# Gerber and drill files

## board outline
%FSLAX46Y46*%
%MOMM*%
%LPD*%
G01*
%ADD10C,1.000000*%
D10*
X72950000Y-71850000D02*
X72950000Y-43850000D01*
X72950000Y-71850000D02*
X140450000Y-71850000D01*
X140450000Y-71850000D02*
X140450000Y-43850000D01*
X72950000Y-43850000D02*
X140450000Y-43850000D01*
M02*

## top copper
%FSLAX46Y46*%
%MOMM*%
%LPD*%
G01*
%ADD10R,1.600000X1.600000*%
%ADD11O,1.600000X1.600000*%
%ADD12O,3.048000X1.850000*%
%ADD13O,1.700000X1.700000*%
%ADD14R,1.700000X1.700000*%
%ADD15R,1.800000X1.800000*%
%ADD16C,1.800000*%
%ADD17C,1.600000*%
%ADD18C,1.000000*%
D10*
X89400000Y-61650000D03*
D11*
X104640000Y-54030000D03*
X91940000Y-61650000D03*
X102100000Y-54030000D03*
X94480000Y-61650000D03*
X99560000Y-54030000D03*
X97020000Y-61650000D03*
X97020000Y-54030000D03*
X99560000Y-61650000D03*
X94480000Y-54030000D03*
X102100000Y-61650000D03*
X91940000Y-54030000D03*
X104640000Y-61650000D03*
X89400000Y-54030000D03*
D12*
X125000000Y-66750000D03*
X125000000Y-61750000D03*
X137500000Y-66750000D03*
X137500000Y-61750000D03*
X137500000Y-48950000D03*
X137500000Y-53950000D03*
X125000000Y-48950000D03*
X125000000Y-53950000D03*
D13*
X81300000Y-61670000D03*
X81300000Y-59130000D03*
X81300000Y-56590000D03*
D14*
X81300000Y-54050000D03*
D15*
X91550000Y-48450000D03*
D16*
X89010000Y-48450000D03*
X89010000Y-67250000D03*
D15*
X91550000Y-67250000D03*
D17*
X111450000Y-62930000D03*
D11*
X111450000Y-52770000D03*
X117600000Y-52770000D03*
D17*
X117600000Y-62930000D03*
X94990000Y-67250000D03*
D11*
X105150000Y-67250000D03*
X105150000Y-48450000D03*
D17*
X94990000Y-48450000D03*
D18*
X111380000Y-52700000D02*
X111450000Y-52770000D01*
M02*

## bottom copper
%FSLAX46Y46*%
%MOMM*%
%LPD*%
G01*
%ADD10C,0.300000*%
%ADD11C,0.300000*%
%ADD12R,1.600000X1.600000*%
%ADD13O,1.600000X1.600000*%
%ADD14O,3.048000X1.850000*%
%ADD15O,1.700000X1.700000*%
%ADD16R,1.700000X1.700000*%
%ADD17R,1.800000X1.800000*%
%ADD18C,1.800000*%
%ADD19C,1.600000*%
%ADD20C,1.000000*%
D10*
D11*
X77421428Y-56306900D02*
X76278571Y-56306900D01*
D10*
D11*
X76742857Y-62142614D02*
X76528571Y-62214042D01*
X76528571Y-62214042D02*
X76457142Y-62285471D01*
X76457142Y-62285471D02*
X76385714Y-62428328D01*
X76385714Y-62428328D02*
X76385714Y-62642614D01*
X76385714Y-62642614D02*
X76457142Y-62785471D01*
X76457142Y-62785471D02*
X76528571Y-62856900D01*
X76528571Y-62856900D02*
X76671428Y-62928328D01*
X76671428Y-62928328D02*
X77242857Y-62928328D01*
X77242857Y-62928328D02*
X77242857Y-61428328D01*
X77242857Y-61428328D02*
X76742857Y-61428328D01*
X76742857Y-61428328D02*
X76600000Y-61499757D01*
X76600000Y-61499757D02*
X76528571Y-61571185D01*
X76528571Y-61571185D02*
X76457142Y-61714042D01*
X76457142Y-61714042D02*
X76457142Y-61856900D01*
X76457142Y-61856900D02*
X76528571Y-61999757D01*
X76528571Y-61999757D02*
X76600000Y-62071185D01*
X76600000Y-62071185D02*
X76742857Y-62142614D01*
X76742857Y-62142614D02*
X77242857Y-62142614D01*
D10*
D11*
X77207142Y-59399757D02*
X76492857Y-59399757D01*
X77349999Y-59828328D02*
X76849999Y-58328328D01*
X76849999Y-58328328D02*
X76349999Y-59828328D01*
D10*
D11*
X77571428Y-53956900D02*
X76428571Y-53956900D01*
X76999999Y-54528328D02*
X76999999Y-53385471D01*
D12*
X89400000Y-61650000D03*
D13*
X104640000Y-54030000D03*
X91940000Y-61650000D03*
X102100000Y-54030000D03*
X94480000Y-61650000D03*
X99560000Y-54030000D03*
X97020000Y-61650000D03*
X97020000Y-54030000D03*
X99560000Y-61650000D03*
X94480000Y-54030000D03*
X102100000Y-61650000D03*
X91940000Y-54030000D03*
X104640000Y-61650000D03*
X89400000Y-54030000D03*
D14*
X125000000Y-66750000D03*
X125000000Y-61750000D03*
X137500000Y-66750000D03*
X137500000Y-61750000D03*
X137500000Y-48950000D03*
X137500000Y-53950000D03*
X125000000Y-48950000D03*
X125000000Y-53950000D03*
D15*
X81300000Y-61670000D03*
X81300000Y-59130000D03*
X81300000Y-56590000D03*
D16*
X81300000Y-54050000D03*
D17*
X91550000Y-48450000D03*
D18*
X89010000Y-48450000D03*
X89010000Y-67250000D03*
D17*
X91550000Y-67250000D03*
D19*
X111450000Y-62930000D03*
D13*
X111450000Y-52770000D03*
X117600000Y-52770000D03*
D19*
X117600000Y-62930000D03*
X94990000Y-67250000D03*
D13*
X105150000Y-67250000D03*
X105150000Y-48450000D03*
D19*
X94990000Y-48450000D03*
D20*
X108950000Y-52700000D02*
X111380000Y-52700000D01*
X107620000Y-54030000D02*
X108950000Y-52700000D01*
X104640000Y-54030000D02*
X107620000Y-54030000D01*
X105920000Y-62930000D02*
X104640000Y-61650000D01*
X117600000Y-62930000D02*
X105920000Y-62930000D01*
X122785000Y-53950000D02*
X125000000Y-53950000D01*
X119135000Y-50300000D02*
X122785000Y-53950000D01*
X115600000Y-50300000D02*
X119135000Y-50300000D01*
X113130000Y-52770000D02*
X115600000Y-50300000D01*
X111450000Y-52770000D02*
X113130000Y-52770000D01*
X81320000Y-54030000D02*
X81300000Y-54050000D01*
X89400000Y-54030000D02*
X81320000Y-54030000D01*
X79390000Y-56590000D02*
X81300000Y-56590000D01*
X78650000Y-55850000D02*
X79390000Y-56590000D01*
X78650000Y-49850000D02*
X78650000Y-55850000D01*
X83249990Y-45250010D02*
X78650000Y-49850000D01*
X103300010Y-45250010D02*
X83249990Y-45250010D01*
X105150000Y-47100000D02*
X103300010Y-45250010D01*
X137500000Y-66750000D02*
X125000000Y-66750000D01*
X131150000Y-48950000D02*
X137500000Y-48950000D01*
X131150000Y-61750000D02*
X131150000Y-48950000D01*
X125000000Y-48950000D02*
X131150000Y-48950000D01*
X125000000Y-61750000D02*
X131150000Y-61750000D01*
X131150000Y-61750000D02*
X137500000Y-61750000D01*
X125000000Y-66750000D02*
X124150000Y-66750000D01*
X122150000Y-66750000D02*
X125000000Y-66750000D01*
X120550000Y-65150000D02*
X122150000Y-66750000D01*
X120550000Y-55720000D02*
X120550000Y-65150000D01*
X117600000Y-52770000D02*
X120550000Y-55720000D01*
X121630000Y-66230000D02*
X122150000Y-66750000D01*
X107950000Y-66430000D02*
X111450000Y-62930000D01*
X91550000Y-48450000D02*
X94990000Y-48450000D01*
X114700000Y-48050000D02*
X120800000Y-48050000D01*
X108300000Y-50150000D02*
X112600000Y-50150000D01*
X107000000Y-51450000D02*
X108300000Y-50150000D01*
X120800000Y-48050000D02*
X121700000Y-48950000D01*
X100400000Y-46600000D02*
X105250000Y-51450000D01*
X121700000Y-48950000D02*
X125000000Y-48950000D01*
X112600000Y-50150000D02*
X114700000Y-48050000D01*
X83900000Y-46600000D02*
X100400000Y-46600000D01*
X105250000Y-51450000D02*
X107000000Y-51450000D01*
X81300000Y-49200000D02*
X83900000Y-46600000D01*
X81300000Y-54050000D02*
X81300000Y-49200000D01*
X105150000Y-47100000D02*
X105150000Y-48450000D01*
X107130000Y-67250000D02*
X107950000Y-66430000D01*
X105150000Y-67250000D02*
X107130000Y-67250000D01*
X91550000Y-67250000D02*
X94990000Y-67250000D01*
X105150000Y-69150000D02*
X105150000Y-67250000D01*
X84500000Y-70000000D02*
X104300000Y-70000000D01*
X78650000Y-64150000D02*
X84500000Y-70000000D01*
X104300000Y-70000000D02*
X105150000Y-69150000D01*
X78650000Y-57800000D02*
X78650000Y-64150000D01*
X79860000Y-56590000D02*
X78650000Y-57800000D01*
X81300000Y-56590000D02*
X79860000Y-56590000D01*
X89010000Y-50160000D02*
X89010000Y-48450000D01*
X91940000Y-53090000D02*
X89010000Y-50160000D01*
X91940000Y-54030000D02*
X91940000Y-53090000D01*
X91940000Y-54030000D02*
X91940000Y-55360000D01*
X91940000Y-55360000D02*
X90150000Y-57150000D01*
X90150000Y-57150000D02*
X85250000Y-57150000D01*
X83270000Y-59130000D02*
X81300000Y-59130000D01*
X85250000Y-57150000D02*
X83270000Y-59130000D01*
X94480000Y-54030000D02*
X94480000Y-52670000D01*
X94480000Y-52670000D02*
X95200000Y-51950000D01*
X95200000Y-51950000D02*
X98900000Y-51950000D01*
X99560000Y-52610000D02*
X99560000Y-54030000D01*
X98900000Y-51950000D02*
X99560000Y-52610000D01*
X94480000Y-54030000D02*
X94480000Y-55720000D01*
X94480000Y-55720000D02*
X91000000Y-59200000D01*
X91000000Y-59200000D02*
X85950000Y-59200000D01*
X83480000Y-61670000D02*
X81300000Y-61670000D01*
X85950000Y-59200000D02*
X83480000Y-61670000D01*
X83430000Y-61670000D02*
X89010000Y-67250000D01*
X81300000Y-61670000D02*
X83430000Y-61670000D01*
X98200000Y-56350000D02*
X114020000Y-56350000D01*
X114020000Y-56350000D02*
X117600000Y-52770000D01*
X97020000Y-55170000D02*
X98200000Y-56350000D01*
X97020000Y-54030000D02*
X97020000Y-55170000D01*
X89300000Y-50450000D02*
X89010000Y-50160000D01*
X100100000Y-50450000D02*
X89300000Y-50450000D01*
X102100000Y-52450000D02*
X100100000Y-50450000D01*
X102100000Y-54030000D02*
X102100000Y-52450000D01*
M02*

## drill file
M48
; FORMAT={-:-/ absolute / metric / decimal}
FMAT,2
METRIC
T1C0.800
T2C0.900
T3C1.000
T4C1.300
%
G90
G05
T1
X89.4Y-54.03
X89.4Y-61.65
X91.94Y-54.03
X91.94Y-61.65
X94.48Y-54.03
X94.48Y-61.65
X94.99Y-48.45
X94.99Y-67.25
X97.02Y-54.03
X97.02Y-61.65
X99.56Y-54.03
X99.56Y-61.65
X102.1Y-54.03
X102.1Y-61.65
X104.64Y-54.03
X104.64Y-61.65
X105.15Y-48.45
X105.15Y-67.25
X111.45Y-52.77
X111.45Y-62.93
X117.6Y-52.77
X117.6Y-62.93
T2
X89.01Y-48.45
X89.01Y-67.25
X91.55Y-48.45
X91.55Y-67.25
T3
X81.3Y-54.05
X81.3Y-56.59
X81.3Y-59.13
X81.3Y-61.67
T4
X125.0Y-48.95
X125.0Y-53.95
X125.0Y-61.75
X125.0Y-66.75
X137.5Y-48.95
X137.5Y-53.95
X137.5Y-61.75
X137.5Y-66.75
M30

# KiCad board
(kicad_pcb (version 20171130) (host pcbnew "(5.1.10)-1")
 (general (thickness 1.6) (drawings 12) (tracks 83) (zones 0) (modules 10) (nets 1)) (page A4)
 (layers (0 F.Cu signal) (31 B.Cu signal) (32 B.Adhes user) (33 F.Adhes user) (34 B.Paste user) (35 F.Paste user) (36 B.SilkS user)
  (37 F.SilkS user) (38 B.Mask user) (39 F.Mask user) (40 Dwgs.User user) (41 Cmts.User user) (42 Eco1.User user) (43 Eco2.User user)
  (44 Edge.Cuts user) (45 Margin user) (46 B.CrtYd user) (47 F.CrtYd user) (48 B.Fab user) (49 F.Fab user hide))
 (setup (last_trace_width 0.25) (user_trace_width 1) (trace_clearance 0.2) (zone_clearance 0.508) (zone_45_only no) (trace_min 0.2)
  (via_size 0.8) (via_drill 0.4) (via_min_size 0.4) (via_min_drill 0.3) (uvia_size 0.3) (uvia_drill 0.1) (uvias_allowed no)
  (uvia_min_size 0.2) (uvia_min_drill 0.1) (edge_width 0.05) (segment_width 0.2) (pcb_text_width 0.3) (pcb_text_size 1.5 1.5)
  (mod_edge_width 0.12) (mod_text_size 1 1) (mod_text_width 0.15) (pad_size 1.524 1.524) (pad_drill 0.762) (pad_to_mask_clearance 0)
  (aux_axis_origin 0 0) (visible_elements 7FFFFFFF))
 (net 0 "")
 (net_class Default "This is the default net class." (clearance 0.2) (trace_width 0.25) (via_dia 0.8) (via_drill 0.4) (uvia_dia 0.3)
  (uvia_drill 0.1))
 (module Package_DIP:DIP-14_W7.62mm (layer F.Cu) (at 89.4 61.65 90)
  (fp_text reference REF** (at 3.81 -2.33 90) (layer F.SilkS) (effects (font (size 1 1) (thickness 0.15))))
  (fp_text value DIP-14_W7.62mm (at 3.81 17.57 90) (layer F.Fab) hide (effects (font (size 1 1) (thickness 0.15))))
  (pad 1 thru_hole rect (at 0 0 90) (size 1.6 1.6) (drill 0.8) (layers *.Cu *.Mask))
  (pad 8 thru_hole oval (at 7.62 15.24 90) (size 1.6 1.6) (drill 0.8) (layers *.Cu *.Mask))
  (pad 2 thru_hole oval (at 0 2.54 90) (size 1.6 1.6) (drill 0.8) (layers *.Cu *.Mask))
  (pad 9 thru_hole oval (at 7.62 12.7 90) (size 1.6 1.6) (drill 0.8) (layers *.Cu *.Mask))
  (pad 3 thru_hole oval (at 0 5.08 90) (size 1.6 1.6) (drill 0.8) (layers *.Cu *.Mask))
  (pad 10 thru_hole oval (at 7.62 10.16 90) (size 1.6 1.6) (drill 0.8) (layers *.Cu *.Mask))
  (pad 4 thru_hole oval (at 0 7.62 90) (size 1.6 1.6) (drill 0.8) (layers *.Cu *.Mask))
  (pad 11 thru_hole oval (at 7.62 7.62 90) (size 1.6 1.6) (drill 0.8) (layers *.Cu *.Mask))
  (pad 5 thru_hole oval (at 0 10.16 90) (size 1.6 1.6) (drill 0.8) (layers *.Cu *.Mask))
  (pad 12 thru_hole oval (at 7.62 5.08 90) (size 1.6 1.6) (drill 0.8) (layers *.Cu *.Mask))
  (pad 6 thru_hole oval (at 0 12.7 90) (size 1.6 1.6) (drill 0.8) (layers *.Cu *.Mask))
  (pad 13 thru_hole oval (at 7.62 2.54 90) (size 1.6 1.6) (drill 0.8) (layers *.Cu *.Mask))
  (pad 7 thru_hole oval (at 0 15.24 90) (size 1.6 1.6) (drill 0.8) (layers *.Cu *.Mask))
  (pad 14 thru_hole oval (at 7.62 0 90) (size 1.6 1.6) (drill 0.8) (layers *.Cu *.Mask)))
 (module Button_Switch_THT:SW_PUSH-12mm (layer F.Cu) (at 137.5 66.75 180)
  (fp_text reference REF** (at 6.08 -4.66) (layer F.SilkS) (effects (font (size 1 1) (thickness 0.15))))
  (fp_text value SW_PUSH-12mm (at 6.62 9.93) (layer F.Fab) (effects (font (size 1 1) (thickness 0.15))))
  (pad 1 thru_hole oval (at 12.5 0 180) (size 3.048 1.85) (drill 1.3) (layers *.Cu *.Mask))
  (pad 2 thru_hole oval (at 12.5 5 180) (size 3.048 1.85) (drill 1.3) (layers *.Cu *.Mask))
  (pad 1 thru_hole oval (at 0 0 180) (size 3.048 1.85) (drill 1.3) (layers *.Cu *.Mask))
  (pad 2 thru_hole oval (at 0 5 180) (size 3.048 1.85) (drill 1.3) (layers *.Cu *.Mask)))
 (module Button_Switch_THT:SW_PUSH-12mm (layer F.Cu) (at 137.5 53.95 180)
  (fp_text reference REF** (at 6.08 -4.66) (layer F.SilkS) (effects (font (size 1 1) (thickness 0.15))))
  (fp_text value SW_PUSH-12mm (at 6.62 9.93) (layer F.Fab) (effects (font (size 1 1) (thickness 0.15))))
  (pad 2 thru_hole oval (at 0 5 180) (size 3.048 1.85) (drill 1.3) (layers *.Cu *.Mask))
  (pad 1 thru_hole oval (at 0 0 180) (size 3.048 1.85) (drill 1.3) (layers *.Cu *.Mask))
  (pad 2 thru_hole oval (at 12.5 5 180) (size 3.048 1.85) (drill 1.3) (layers *.Cu *.Mask))
  (pad 1 thru_hole oval (at 12.5 0 180) (size 3.048 1.85) (drill 1.3) (layers *.Cu *.Mask)))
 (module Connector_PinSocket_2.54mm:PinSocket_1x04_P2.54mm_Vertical (layer F.Cu) (at 81.3 54.05)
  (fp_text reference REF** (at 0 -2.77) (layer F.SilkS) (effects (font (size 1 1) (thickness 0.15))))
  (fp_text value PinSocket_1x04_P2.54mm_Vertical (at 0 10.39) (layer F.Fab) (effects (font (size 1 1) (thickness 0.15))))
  (pad 4 thru_hole oval (at 0 7.62) (size 1.7 1.7) (drill 1) (layers *.Cu *.Mask))
  (pad 3 thru_hole oval (at 0 5.08) (size 1.7 1.7) (drill 1) (layers *.Cu *.Mask))
  (pad 2 thru_hole oval (at 0 2.54) (size 1.7 1.7) (drill 1) (layers *.Cu *.Mask))
  (pad 1 thru_hole rect (at 0 0) (size 1.7 1.7) (drill 1) (layers *.Cu *.Mask)))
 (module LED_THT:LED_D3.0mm (layer F.Cu) (at 91.55 48.45 180)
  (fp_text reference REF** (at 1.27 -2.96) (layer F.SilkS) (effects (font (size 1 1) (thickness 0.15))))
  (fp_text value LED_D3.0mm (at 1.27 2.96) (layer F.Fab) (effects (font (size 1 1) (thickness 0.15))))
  (pad 1 thru_hole rect (at 0 0 180) (size 1.8 1.8) (drill 0.9) (layers *.Cu *.Mask))
  (pad 2 thru_hole circle (at 2.54 0 180) (size 1.8 1.8) (drill 0.9) (layers *.Cu *.Mask)))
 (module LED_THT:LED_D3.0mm (layer F.Cu) (at 91.55 67.25 180)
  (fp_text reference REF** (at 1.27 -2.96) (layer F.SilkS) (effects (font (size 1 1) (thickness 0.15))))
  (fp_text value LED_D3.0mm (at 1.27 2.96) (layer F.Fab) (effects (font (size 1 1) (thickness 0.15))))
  (pad 2 thru_hole circle (at 2.54 0 180) (size 1.8 1.8) (drill 0.9) (layers *.Cu *.Mask))
  (pad 1 thru_hole rect (at 0 0 180) (size 1.8 1.8) (drill 0.9) (layers *.Cu *.Mask)))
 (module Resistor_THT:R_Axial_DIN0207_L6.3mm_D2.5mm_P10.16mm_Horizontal (layer F.Cu) (at 111.45 62.93 90)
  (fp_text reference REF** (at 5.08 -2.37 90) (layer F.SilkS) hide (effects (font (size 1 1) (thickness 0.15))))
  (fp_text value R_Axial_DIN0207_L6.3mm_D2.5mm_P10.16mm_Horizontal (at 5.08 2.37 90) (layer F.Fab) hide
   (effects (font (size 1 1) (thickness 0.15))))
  (pad 1 thru_hole circle (at 0 0 90) (size 1.6 1.6) (drill 0.8) (layers *.Cu *.Mask))
  (pad 2 thru_hole oval (at 10.16 0 90) (size 1.6 1.6) (drill 0.8) (layers *.Cu *.Mask)))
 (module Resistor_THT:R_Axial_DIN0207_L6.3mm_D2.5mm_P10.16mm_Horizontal (layer F.Cu) (at 117.6 62.93 90)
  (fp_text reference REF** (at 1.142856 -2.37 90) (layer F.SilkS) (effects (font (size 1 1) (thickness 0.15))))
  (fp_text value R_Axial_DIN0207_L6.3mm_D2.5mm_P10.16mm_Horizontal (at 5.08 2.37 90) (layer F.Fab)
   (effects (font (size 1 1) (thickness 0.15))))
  (pad 2 thru_hole oval (at 10.16 0 90) (size 1.6 1.6) (drill 0.8) (layers *.Cu *.Mask))
  (pad 1 thru_hole circle (at 0 0 90) (size 1.6 1.6) (drill 0.8) (layers *.Cu *.Mask)))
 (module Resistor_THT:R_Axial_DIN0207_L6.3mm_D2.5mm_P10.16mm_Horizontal (layer F.Cu) (at 94.99 67.25)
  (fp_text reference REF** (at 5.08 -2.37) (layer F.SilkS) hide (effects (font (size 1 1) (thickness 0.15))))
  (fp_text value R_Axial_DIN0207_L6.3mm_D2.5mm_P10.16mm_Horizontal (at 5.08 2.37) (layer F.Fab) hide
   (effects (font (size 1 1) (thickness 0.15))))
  (pad 1 thru_hole circle (at 0 0) (size 1.6 1.6) (drill 0.8) (layers *.Cu *.Mask))
  (pad 2 thru_hole oval (at 10.16 0) (size 1.6 1.6) (drill 0.8) (layers *.Cu *.Mask)))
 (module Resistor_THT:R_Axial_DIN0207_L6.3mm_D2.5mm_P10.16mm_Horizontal (layer F.Cu) (at 94.99 48.45)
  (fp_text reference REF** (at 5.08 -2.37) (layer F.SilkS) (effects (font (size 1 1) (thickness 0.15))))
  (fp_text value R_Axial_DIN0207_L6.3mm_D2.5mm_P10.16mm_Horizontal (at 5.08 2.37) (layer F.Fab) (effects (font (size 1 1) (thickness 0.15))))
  (pad 2 thru_hole oval (at 10.16 0) (size 1.6 1.6) (drill 0.8) (layers *.Cu *.Mask))
  (pad 1 thru_hole circle (at 0 0) (size 1.6 1.6) (drill 0.8) (layers *.Cu *.Mask)))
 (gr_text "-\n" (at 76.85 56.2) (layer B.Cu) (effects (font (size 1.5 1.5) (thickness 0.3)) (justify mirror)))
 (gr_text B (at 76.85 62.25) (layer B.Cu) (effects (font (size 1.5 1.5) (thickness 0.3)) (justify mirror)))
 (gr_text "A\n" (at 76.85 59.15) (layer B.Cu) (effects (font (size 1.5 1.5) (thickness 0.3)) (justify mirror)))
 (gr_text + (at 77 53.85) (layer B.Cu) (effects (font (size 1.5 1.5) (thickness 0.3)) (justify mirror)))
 (gr_line (start 72.95 71.85) (end 72.95 43.85) (layer Edge.Cuts) (width 1))
 (gr_line (start 72.95 71.85) (end 140.45 71.85) (layer Edge.Cuts) (width 1))
 (gr_line (start 140.45 71.85) (end 140.45 43.85) (layer Edge.Cuts) (width 1))
 (gr_line (start 72.95 43.85) (end 140.45 43.85) (layer Edge.Cuts) (width 1))
 (segment (start 111.38 52.7) (end 111.45 52.77) (width 1) (layer F.Cu) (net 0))
 (segment (start 108.95 52.7) (end 111.38 52.7) (width 1) (layer B.Cu) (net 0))
 (segment (start 107.62 54.03) (end 108.95 52.7) (width 1) (layer B.Cu) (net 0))
 (segment (start 104.64 54.03) (end 107.62 54.03) (width 1) (layer B.Cu) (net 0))
 (segment (start 105.92 62.93) (end 104.64 61.65) (width 1) (layer B.Cu) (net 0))
 (segment (start 117.6 62.93) (end 105.92 62.93) (width 1) (layer B.Cu) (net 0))
 (segment (start 122.785 53.95) (end 125 53.95) (width 1) (layer B.Cu) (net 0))
 (segment (start 119.135 50.3) (end 122.785 53.95) (width 1) (layer B.Cu) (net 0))
 (segment (start 115.6 50.3) (end 119.135 50.3) (width 1) (layer B.Cu) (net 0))
 (segment (start 113.13 52.77) (end 115.6 50.3) (width 1) (layer B.Cu) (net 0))
 (segment (start 111.45 52.77) (end 113.13 52.77) (width 1) (layer B.Cu) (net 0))
 (segment (start 81.32 54.03) (end 81.3 54.05) (width 1) (layer B.Cu) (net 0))
 (segment (start 89.4 54.03) (end 81.32 54.03) (width 1) (layer B.Cu) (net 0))
 (segment (start 79.39 56.59) (end 81.3 56.59) (width 1) (layer B.Cu) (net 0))
 (segment (start 78.65 55.85) (end 79.39 56.59) (width 1) (layer B.Cu) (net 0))
 (segment (start 78.65 49.85) (end 78.65 55.85) (width 1) (layer B.Cu) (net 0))
 (segment (start 83.24999 45.25001) (end 78.65 49.85) (width 1) (layer B.Cu) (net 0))
 (segment (start 103.30001 45.25001) (end 83.24999 45.25001) (width 1) (layer B.Cu) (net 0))
 (segment (start 105.15 47.1) (end 103.30001 45.25001) (width 1) (layer B.Cu) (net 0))
 (segment (start 137.5 66.75) (end 125 66.75) (width 1) (layer B.Cu) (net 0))
 (segment (start 131.15 48.95) (end 137.5 48.95) (width 1) (layer B.Cu) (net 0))
 (segment (start 131.15 61.75) (end 131.15 48.95) (width 1) (layer B.Cu) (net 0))
 (segment (start 125 48.95) (end 131.15 48.95) (width 1) (layer B.Cu) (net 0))
 (segment (start 125 61.75) (end 131.15 61.75) (width 1) (layer B.Cu) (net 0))
 (segment (start 131.15 61.75) (end 137.5 61.75) (width 1) (layer B.Cu) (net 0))
 (segment (start 125 66.75) (end 124.15 66.75) (width 1) (layer B.Cu) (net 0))
 (segment (start 122.15 66.75) (end 125 66.75) (width 1) (layer B.Cu) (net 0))
 (segment (start 120.55 65.15) (end 122.15 66.75) (width 1) (layer B.Cu) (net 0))
 (segment (start 120.55 55.72) (end 120.55 65.15) (width 1) (layer B.Cu) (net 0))
 (segment (start 117.6 52.77) (end 120.55 55.72) (width 1) (layer B.Cu) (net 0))
 (segment (start 121.63 66.23) (end 122.15 66.75) (width 1) (layer B.Cu) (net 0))
 (segment (start 107.95 66.43) (end 111.45 62.93) (width 1) (layer B.Cu) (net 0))
 (segment (start 91.55 48.45) (end 94.99 48.45) (width 1) (layer B.Cu) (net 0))
 (segment (start 114.7 48.05) (end 120.8 48.05) (width 1) (layer B.Cu) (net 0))
 (segment (start 108.3 50.15) (end 112.6 50.15) (width 1) (layer B.Cu) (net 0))
 (segment (start 107 51.45) (end 108.3 50.15) (width 1) (layer B.Cu) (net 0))
 (segment (start 120.8 48.05) (end 121.7 48.95) (width 1) (layer B.Cu) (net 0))
 (segment (start 100.4 46.6) (end 105.25 51.45) (width 1) (layer B.Cu) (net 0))
 (segment (start 121.7 48.95) (end 125 48.95) (width 1) (layer B.Cu) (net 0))
 (segment (start 112.6 50.15) (end 114.7 48.05) (width 1) (layer B.Cu) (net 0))
 (segment (start 83.9 46.6) (end 100.4 46.6) (width 1) (layer B.Cu) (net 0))
 (segment (start 105.25 51.45) (end 107 51.45) (width 1) (layer B.Cu) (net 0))
 (segment (start 81.3 49.2) (end 83.9 46.6) (width 1) (layer B.Cu) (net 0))
 (segment (start 81.3 54.05) (end 81.3 49.2) (width 1) (layer B.Cu) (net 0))
 (segment (start 105.15 47.1) (end 105.15 48.45) (width 1) (layer B.Cu) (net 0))
 (segment (start 107.13 67.25) (end 107.95 66.43) (width 1) (layer B.Cu) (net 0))
 (segment (start 105.15 67.25) (end 107.13 67.25) (width 1) (layer B.Cu) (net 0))
 (segment (start 91.55 67.25) (end 94.99 67.25) (width 1) (layer B.Cu) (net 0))
 (segment (start 105.15 69.15) (end 105.15 67.25) (width 1) (layer B.Cu) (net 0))
 (segment (start 84.5 70) (end 104.3 70) (width 1) (layer B.Cu) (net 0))
 (segment (start 78.65 64.15) (end 84.5 70) (width 1) (layer B.Cu) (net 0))
 (segment (start 104.3 70) (end 105.15 69.15) (width 1) (layer B.Cu) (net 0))
 (segment (start 78.65 57.8) (end 78.65 64.15) (width 1) (layer B.Cu) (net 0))
 (segment (start 79.86 56.59) (end 78.65 57.8) (width 1) (layer B.Cu) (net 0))
 (segment (start 81.3 56.59) (end 79.86 56.59) (width 1) (layer B.Cu) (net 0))
 (segment (start 89.01 50.16) (end 89.01 48.45) (width 1) (layer B.Cu) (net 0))
 (segment (start 91.94 53.09) (end 89.01 50.16) (width 1) (layer B.Cu) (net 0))
 (segment (start 91.94 54.03) (end 91.94 53.09) (width 1) (layer B.Cu) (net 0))
 (segment (start 91.94 54.03) (end 91.94 55.36) (width 1) (layer B.Cu) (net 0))
 (segment (start 91.94 55.36) (end 90.15 57.15) (width 1) (layer B.Cu) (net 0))
 (segment (start 90.15 57.15) (end 85.25 57.15) (width 1) (layer B.Cu) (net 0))
 (segment (start 83.27 59.13) (end 81.3 59.13) (width 1) (layer B.Cu) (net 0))
 (segment (start 85.25 57.15) (end 83.27 59.13) (width 1) (layer B.Cu) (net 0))
 (segment (start 94.48 54.03) (end 94.48 52.67) (width 1) (layer B.Cu) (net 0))
 (segment (start 94.48 52.67) (end 95.2 51.95) (width 1) (layer B.Cu) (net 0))
 (segment (start 95.2 51.95) (end 98.9 51.95) (width 1) (layer B.Cu) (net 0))
 (segment (start 99.56 52.61) (end 99.56 54.03) (width 1) (layer B.Cu) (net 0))
 (segment (start 98.9 51.95) (end 99.56 52.61) (width 1) (layer B.Cu) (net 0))
 (segment (start 94.48 54.03) (end 94.48 55.72) (width 1) (layer B.Cu) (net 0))
 (segment (start 94.48 55.72) (end 91 59.2) (width 1) (layer B.Cu) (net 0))
 (segment (start 91 59.2) (end 85.95 59.2) (width 1) (layer B.Cu) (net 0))
 (segment (start 83.48 61.67) (end 81.3 61.67) (width 1) (layer B.Cu) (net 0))
 (segment (start 85.95 59.2) (end 83.48 61.67) (width 1) (layer B.Cu) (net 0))
 (segment (start 83.43 61.67) (end 89.01 67.25) (width 1) (layer B.Cu) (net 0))
 (segment (start 81.3 61.67) (end 83.43 61.67) (width 1) (layer B.Cu) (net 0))
 (segment (start 98.2 56.35) (end 114.02 56.35) (width 1) (layer B.Cu) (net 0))
 (segment (start 114.02 56.35) (end 117.6 52.77) (width 1) (layer B.Cu) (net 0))
 (segment (start 97.02 55.17) (end 98.2 56.35) (width 1) (layer B.Cu) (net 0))
 (segment (start 97.02 54.03) (end 97.02 55.17) (width 1) (layer B.Cu) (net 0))
 (segment (start 89.3 50.45) (end 89.01 50.16) (width 1) (layer B.Cu) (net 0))
 (segment (start 100.1 50.45) (end 89.3 50.45) (width 1) (layer B.Cu) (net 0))
 (segment (start 102.1 52.45) (end 100.1 50.45) (width 1) (layer B.Cu) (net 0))
 (segment (start 102.1 54.03) (end 102.1 52.45) (width 1) (layer B.Cu) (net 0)))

